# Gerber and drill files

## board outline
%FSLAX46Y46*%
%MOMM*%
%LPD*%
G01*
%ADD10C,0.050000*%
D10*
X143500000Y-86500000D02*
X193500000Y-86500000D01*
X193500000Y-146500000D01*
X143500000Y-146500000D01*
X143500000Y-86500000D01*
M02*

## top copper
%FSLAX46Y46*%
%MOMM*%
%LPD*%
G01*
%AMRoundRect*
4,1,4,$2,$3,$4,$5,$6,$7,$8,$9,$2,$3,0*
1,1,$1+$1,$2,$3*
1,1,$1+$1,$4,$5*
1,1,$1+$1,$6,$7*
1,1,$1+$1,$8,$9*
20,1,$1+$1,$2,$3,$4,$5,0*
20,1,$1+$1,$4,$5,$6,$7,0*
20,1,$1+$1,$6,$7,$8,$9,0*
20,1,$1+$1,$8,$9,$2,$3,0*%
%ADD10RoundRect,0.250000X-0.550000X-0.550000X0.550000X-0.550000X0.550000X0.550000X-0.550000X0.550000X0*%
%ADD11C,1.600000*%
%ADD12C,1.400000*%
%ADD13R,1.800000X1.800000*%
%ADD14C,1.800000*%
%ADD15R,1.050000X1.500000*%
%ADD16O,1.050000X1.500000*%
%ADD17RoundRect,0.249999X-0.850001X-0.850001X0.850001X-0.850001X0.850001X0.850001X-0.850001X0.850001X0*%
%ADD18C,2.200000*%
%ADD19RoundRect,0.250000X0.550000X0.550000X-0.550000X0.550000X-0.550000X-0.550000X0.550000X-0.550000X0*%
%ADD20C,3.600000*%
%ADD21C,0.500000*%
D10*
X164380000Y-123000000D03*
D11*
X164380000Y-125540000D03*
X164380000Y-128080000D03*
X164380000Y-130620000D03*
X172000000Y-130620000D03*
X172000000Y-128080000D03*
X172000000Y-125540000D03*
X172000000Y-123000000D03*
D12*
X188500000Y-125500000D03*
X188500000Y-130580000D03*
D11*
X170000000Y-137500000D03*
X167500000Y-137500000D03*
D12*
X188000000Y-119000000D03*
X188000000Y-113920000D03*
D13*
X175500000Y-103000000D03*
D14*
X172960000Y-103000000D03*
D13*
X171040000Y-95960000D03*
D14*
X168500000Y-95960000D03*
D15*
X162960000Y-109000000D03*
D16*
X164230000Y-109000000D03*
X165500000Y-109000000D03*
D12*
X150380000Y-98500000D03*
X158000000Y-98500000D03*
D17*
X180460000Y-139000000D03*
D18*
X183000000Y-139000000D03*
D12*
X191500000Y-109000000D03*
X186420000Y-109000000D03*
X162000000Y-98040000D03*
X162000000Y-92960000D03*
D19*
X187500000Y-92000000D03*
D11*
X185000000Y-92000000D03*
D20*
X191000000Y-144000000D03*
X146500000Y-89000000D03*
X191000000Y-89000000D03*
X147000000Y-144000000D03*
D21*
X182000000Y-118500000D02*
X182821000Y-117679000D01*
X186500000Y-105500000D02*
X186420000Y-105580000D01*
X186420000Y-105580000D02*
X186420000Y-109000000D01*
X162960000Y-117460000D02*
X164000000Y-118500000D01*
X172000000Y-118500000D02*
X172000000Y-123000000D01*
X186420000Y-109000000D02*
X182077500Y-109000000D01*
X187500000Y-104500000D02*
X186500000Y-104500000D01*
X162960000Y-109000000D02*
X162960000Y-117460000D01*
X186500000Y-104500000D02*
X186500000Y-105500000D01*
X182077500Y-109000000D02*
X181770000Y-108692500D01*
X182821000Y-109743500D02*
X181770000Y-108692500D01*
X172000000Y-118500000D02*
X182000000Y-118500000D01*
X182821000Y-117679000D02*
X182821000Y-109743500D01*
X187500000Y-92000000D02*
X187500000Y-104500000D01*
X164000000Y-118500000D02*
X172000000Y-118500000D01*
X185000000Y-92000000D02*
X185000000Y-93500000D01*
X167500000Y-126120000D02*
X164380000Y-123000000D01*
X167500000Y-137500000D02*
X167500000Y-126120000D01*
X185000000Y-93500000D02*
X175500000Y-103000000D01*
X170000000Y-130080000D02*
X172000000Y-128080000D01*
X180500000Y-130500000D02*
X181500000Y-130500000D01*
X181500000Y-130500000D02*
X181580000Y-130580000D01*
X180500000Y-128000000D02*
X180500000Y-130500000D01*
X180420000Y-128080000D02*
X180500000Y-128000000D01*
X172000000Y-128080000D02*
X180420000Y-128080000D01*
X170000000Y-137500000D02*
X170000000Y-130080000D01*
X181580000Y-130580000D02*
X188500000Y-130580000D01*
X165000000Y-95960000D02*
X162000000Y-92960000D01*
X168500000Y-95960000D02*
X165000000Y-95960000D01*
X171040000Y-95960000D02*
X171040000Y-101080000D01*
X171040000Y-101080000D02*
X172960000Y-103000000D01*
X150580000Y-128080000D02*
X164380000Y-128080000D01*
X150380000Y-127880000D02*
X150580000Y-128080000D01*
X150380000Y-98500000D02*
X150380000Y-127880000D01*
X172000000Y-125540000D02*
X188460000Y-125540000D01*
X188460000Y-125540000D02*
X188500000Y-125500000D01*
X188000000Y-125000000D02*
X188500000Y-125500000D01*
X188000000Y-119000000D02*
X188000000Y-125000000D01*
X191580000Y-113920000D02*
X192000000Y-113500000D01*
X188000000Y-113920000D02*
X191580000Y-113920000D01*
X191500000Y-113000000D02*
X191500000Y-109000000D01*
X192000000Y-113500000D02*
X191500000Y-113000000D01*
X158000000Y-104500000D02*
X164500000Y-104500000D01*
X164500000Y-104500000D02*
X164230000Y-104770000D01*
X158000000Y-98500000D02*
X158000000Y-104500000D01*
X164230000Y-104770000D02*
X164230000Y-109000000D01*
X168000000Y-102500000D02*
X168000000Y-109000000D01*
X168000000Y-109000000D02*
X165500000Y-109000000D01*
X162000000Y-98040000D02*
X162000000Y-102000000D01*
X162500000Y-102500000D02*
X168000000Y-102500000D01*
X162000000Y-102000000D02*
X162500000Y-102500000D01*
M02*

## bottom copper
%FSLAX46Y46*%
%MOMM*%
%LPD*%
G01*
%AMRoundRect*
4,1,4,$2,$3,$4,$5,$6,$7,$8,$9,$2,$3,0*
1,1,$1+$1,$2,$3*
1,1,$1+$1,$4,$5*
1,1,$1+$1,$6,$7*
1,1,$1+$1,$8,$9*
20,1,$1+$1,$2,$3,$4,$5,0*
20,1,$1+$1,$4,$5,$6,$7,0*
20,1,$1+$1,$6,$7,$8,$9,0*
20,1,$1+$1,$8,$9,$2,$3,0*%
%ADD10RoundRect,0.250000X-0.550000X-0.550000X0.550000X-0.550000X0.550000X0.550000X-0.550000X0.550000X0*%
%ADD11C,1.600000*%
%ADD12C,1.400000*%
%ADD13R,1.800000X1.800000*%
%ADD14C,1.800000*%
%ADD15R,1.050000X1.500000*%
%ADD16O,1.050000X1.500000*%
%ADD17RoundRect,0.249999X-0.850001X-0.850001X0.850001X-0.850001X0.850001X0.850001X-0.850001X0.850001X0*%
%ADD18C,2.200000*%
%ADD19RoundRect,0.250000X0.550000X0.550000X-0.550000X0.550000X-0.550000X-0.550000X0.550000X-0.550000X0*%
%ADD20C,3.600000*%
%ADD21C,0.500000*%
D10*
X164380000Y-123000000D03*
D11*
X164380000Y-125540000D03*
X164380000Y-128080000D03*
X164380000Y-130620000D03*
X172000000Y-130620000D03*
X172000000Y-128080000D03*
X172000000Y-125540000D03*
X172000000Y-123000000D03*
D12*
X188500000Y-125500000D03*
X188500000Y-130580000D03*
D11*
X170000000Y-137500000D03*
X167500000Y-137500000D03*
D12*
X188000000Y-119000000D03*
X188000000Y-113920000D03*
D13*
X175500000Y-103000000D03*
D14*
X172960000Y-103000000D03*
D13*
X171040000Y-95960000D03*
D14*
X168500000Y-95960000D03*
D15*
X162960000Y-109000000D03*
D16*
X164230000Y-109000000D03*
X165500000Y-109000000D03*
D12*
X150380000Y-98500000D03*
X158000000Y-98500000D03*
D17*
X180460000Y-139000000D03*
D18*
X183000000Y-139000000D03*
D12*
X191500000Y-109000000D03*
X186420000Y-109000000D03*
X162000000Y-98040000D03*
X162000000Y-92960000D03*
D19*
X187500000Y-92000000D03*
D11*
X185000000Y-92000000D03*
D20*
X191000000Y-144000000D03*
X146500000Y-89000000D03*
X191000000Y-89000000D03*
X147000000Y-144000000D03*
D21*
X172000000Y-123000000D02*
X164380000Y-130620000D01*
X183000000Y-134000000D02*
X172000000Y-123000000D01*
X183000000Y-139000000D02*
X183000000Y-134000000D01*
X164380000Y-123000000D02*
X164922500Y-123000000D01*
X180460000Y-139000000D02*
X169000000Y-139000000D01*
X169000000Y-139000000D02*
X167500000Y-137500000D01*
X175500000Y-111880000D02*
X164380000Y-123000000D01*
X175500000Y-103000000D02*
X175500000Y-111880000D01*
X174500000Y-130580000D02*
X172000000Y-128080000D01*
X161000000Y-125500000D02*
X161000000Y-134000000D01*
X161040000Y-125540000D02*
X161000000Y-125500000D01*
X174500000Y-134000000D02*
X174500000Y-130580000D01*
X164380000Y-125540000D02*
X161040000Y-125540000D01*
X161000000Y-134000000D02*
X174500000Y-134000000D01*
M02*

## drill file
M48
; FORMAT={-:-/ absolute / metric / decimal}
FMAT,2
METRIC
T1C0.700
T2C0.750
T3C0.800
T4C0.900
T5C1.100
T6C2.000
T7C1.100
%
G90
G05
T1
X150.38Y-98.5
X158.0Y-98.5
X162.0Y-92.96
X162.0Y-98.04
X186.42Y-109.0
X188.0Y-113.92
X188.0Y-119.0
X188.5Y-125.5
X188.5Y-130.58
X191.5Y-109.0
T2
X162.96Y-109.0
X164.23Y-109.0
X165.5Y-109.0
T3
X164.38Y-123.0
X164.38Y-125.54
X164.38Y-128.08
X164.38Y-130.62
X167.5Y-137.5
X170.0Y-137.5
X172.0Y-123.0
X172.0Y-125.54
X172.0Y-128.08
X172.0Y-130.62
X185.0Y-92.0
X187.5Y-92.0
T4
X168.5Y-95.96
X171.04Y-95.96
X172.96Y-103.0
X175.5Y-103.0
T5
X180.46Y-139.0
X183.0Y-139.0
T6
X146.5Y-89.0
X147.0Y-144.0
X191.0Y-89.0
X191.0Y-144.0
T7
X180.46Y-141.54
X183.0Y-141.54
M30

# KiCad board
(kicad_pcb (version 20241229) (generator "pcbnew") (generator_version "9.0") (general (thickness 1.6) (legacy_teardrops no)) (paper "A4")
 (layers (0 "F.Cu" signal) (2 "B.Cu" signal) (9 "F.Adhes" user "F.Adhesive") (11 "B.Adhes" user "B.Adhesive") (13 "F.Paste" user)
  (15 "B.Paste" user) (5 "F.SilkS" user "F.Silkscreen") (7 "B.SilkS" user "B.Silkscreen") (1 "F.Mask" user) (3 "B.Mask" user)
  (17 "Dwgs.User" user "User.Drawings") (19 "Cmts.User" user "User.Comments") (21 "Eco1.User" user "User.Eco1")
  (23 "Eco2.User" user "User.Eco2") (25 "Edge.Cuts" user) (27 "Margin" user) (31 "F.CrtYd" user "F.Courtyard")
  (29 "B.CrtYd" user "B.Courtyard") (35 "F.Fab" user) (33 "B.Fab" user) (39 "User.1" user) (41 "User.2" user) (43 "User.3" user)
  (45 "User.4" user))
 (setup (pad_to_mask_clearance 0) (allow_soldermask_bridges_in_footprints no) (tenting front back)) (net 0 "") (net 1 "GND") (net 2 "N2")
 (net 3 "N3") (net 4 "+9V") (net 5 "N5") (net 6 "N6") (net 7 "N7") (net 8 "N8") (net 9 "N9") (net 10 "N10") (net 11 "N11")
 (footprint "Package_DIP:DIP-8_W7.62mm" (layer "F.Cu") (at 164.38 123)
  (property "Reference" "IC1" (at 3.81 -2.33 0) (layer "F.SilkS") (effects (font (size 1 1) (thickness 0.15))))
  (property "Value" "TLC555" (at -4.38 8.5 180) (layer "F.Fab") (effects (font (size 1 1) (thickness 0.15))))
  (pad "1" thru_hole roundrect (at 0 0) (size 1.6 1.6) (drill 0.8) (layers "*.Cu" "*.Mask") (remove_unused_layers no)
   (roundrect_rratio 0.15625) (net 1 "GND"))
  (pad "2" thru_hole circle (at 0 2.54) (size 1.6 1.6) (drill 0.8) (layers "*.Cu" "*.Mask") (remove_unused_layers no) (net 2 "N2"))
  (pad "3" thru_hole circle (at 0 5.08) (size 1.6 1.6) (drill 0.8) (layers "*.Cu" "*.Mask") (remove_unused_layers no) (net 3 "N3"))
  (pad "4" thru_hole circle (at 0 7.62) (size 1.6 1.6) (drill 0.8) (layers "*.Cu" "*.Mask") (remove_unused_layers no) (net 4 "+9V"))
  (pad "5" thru_hole circle (at 7.62 7.62) (size 1.6 1.6) (drill 0.8) (layers "*.Cu" "*.Mask") (remove_unused_layers no) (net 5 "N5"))
  (pad "6" thru_hole circle (at 7.62 5.08) (size 1.6 1.6) (drill 0.8) (layers "*.Cu" "*.Mask") (remove_unused_layers no) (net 2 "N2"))
  (pad "7" thru_hole circle (at 7.62 2.54) (size 1.6 1.6) (drill 0.8) (layers "*.Cu" "*.Mask") (remove_unused_layers no) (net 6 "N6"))
  (pad "8" thru_hole circle (at 7.62 0) (size 1.6 1.6) (drill 0.8) (layers "*.Cu" "*.Mask") (remove_unused_layers no) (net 4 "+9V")))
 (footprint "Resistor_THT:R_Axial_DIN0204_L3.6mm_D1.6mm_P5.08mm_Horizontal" (layer "F.Cu") (at 188.5 125.5 -90)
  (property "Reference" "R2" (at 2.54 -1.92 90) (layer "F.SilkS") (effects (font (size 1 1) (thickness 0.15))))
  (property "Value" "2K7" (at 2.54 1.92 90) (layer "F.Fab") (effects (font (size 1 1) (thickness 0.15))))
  (pad "1" thru_hole circle (at 0 0 270) (size 1.4 1.4) (drill 0.7) (layers "*.Cu" "*.Mask") (remove_unused_layers no) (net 6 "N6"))
  (pad "2" thru_hole circle (at 5.08 0 270) (size 1.4 1.4) (drill 0.7) (layers "*.Cu" "*.Mask") (remove_unused_layers no) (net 2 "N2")))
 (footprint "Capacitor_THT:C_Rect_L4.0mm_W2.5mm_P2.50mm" (layer "F.Cu") (at 170 137.5 180)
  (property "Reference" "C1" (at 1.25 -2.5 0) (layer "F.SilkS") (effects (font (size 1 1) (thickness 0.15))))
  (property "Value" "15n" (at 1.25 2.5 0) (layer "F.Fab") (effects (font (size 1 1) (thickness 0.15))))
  (pad "1" thru_hole circle (at 0 0 180) (size 1.6 1.6) (drill 0.8) (layers "*.Cu" "*.Mask") (remove_unused_layers no) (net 2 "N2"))
  (pad "2" thru_hole circle (at 2.5 0 180) (size 1.6 1.6) (drill 0.8) (layers "*.Cu" "*.Mask") (remove_unused_layers no) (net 1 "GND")))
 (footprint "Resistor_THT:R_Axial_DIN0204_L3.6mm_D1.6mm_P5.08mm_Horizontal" (layer "F.Cu") (at 188 119 90)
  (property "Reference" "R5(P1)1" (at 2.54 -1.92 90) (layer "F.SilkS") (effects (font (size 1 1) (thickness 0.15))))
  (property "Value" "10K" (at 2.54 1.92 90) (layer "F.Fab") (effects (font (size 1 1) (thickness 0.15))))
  (pad "1" thru_hole circle (at 0 0 90) (size 1.4 1.4) (drill 0.7) (layers "*.Cu" "*.Mask") (remove_unused_layers no) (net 6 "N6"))
  (pad "2" thru_hole circle (at 5.08 0 90) (size 1.4 1.4) (drill 0.7) (layers "*.Cu" "*.Mask") (remove_unused_layers no) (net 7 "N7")))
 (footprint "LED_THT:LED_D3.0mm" (layer "F.Cu") (at 175.5 103 180)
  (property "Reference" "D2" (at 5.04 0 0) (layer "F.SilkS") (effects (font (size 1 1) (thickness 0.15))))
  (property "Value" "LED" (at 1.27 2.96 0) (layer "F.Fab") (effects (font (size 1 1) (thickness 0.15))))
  (pad "1" thru_hole rect (at 0 0 180) (size 1.8 1.8) (drill 0.9) (layers "*.Cu" "*.Mask") (remove_unused_layers no) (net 1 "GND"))
  (pad "2" thru_hole circle (at 2.54 0 180) (size 1.8 1.8) (drill 0.9) (layers "*.Cu" "*.Mask") (remove_unused_layers no) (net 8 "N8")))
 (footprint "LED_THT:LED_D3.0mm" (layer "F.Cu") (at 171.04 95.96 180)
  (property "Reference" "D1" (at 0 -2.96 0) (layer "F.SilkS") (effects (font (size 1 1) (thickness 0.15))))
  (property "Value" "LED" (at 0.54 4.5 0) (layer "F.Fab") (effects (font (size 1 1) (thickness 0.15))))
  (pad "1" thru_hole rect (at 0 0 180) (size 1.8 1.8) (drill 0.9) (layers "*.Cu" "*.Mask") (remove_unused_layers no) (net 8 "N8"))
  (pad "2" thru_hole circle (at 2.54 0 180) (size 1.8 1.8) (drill 0.9) (layers "*.Cu" "*.Mask") (remove_unused_layers no) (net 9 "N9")))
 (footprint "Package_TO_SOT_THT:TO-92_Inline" (layer "F.Cu") (at 162.96 109)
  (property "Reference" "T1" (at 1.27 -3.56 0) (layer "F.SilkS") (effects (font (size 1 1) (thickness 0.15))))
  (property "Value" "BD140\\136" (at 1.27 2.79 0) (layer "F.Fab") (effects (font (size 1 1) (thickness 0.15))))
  (pad "1" thru_hole rect (at 0 0) (size 1.05 1.5) (drill 0.75) (layers "*.Cu" "*.Mask") (remove_unused_layers no) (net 4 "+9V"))
  (pad "2" thru_hole oval (at 1.27 0) (size 1.05 1.5) (drill 0.75) (layers "*.Cu" "*.Mask") (remove_unused_layers no) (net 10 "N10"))
  (pad "3" thru_hole oval (at 2.54 0) (size 1.05 1.5) (drill 0.75) (layers "*.Cu" "*.Mask") (remove_unused_layers no) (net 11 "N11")))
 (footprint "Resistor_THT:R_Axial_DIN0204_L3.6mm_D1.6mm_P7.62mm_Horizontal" (layer "F.Cu") (at 150.38 98.5)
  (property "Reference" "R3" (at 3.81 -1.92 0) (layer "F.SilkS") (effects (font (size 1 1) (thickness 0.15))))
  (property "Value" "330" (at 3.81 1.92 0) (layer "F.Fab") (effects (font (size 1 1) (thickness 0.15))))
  (pad "1" thru_hole circle (at 0 0) (size 1.4 1.4) (drill 0.7) (layers "*.Cu" "*.Mask") (remove_unused_layers no) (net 3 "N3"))
  (pad "2" thru_hole circle (at 7.62 0) (size 1.4 1.4) (drill 0.7) (layers "*.Cu" "*.Mask") (remove_unused_layers no) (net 10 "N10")))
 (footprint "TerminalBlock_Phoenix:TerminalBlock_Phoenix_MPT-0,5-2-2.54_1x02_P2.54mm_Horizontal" (layer "F.Cu") (at 180.46 139)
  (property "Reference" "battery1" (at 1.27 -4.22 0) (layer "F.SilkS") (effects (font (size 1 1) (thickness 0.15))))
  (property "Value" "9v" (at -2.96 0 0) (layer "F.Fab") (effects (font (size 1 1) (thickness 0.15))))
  (pad "" np_thru_hole circle (at 0 2.54) (size 1.1 1.1) (drill 1.1) (layers "*.Cu" "*.Mask"))
  (pad "" np_thru_hole circle (at 2.54 2.54) (size 1.1 1.1) (drill 1.1) (layers "*.Cu" "*.Mask"))
  (pad "1" thru_hole roundrect (at 0 0) (size 2.2 2.2) (drill 1.1) (layers "*.Cu" "*.Mask") (remove_unused_layers no)
   (roundrect_rratio 0.113636) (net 1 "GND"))
  (pad "2" thru_hole circle (at 2.54 0) (size 2.2 2.2) (drill 1.1) (layers "*.Cu" "*.Mask") (remove_unused_layers no) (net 4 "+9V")))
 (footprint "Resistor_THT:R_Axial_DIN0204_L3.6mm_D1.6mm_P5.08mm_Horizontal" (layer "F.Cu") (at 191.5 109 180)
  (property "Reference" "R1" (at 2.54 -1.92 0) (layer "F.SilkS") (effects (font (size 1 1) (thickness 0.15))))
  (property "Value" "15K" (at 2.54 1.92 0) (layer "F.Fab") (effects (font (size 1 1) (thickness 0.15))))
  (pad "1" thru_hole circle (at 0 0 180) (size 1.4 1.4) (drill 0.7) (layers "*.Cu" "*.Mask") (remove_unused_layers no) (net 7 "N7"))
  (pad "2" thru_hole circle (at 5.08 0 180) (size 1.4 1.4) (drill 0.7) (layers "*.Cu" "*.Mask") (remove_unused_layers no) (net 4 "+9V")))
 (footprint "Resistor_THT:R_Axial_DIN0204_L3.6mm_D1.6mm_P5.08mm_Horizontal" (layer "F.Cu") (at 162 98.04 90)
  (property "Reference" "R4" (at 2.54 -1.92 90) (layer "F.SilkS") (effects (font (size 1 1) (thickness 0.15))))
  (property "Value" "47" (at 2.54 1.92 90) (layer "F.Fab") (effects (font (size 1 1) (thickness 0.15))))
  (pad "1" thru_hole circle (at 0 0 90) (size 1.4 1.4) (drill 0.7) (layers "*.Cu" "*.Mask") (remove_unused_layers no) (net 11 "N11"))
  (pad "2" thru_hole circle (at 5.08 0 90) (size 1.4 1.4) (drill 0.7) (layers "*.Cu" "*.Mask") (remove_unused_layers no) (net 9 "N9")))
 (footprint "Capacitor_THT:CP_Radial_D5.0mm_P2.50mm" (layer "F.Cu") (at 187.5 92 180)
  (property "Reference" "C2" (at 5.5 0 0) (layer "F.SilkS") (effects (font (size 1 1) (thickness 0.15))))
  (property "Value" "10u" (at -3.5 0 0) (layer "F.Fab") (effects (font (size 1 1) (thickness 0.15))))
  (pad "1" thru_hole roundrect (at 0 0 180) (size 1.6 1.6) (drill 0.8) (layers "*.Cu" "*.Mask") (remove_unused_layers no)
   (roundrect_rratio 0.15625) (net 4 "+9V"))
  (pad "2" thru_hole circle (at 2.5 0 180) (size 1.6 1.6) (drill 0.8) (layers "*.Cu" "*.Mask") (remove_unused_layers no) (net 1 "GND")))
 (gr_rect (start 143.5 86.5) (end 193.5 146.5) (stroke (width 0.05) (type default)) (fill no) (layer "Edge.Cuts"))
 (via (at 191 144) (size 3.6) (drill 2) (layers "F.Cu" "B.Cu") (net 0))
 (via (at 146.5 89) (size 3.6) (drill 2) (layers "F.Cu" "B.Cu") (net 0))
 (via (at 191 89) (size 3.6) (drill 2) (layers "F.Cu" "B.Cu") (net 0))
 (via (at 147 144) (size 3.6) (drill 2) (layers "F.Cu" "B.Cu") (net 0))
 (segment (start 182 118.5) (end 182.821 117.679) (width 0.5) (layer "F.Cu") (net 4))
 (segment (start 186.5 105.5) (end 186.42 105.58) (width 0.5) (layer "F.Cu") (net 4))
 (segment (start 186.42 105.58) (end 186.42 109) (width 0.5) (layer "F.Cu") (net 4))
 (segment (start 162.96 117.46) (end 164 118.5) (width 0.5) (layer "F.Cu") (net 4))
 (segment (start 172 118.5) (end 172 123) (width 0.5) (layer "F.Cu") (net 4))
 (segment (start 186.42 109) (end 182.0775 109) (width 0.5) (layer "F.Cu") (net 4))
 (segment (start 187.5 104.5) (end 186.5 104.5) (width 0.5) (layer "F.Cu") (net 4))
 (segment (start 162.96 109) (end 162.96 117.46) (width 0.5) (layer "F.Cu") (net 4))
 (segment (start 186.5 104.5) (end 186.5 105.5) (width 0.5) (layer "F.Cu") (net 4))
 (segment (start 182.0775 109) (end 181.77 108.6925) (width 0.5) (layer "F.Cu") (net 4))
 (segment (start 182.821 109.7435) (end 181.77 108.6925) (width 0.5) (layer "F.Cu") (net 4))
 (segment (start 172 118.5) (end 182 118.5) (width 0.5) (layer "F.Cu") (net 4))
 (segment (start 182.821 117.679) (end 182.821 109.7435) (width 0.5) (layer "F.Cu") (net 4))
 (segment (start 187.5 92) (end 187.5 104.5) (width 0.5) (layer "F.Cu") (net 4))
 (segment (start 164 118.5) (end 172 118.5) (width 0.5) (layer "F.Cu") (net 4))
 (segment (start 172 123) (end 164.38 130.62) (width 0.5) (layer "B.Cu") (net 4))
 (segment (start 183 134) (end 172 123) (width 0.5) (layer "B.Cu") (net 4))
 (segment (start 183 139) (end 183 134) (width 0.5) (layer "B.Cu") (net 4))
 (segment (start 185 92) (end 185 93.5) (width 0.5) (layer "F.Cu") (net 1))
 (segment (start 167.5 126.12) (end 164.38 123) (width 0.5) (layer "F.Cu") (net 1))
 (segment (start 167.5 137.5) (end 167.5 126.12) (width 0.5) (layer "F.Cu") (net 1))
 (segment (start 185 93.5) (end 175.5 103) (width 0.5) (layer "F.Cu") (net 1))
 (segment (start 164.38 123) (end 164.9225 123) (width 0.5) (layer "B.Cu") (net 1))
 (segment (start 180.46 139) (end 169 139) (width 0.5) (layer "B.Cu") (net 1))
 (segment (start 169 139) (end 167.5 137.5) (width 0.5) (layer "B.Cu") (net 1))
 (segment (start 175.5 111.88) (end 164.38 123) (width 0.5) (layer "B.Cu") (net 1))
 (segment (start 175.5 103) (end 175.5 111.88) (width 0.5) (layer "B.Cu") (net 1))
 (segment (start 170 130.08) (end 172 128.08) (width 0.5) (layer "F.Cu") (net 2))
 (segment (start 180.5 130.5) (end 181.5 130.5) (width 0.5) (layer "F.Cu") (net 2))
 (segment (start 181.5 130.5) (end 181.58 130.58) (width 0.5) (layer "F.Cu") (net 2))
 (segment (start 180.5 128) (end 180.5 130.5) (width 0.5) (layer "F.Cu") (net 2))
 (segment (start 180.42 128.08) (end 180.5 128) (width 0.5) (layer "F.Cu") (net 2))
 (segment (start 172 128.08) (end 180.42 128.08) (width 0.5) (layer "F.Cu") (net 2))
 (segment (start 170 137.5) (end 170 130.08) (width 0.5) (layer "F.Cu") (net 2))
 (segment (start 181.58 130.58) (end 188.5 130.58) (width 0.5) (layer "F.Cu") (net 2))
 (segment (start 174.5 130.58) (end 172 128.08) (width 0.5) (layer "B.Cu") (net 2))
 (segment (start 161 125.5) (end 161 134) (width 0.5) (layer "B.Cu") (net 2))
 (segment (start 161.04 125.54) (end 161 125.5) (width 0.5) (layer "B.Cu") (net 2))
 (segment (start 174.5 134) (end 174.5 130.58) (width 0.5) (layer "B.Cu") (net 2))
 (segment (start 164.38 125.54) (end 161.04 125.54) (width 0.5) (layer "B.Cu") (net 2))
 (segment (start 161 134) (end 174.5 134) (width 0.5) (layer "B.Cu") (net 2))
 (segment (start 165 95.96) (end 162 92.96) (width 0.5) (layer "F.Cu") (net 9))
 (segment (start 168.5 95.96) (end 165 95.96) (width 0.5) (layer "F.Cu") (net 9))
 (segment (start 171.04 95.96) (end 171.04 101.08) (width 0.5) (layer "F.Cu") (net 8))
 (segment (start 171.04 101.08) (end 172.96 103) (width 0.5) (layer "F.Cu") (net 8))
 (segment (start 150.58 128.08) (end 164.38 128.08) (width 0.5) (layer "F.Cu") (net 3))
 (segment (start 150.38 127.88) (end 150.58 128.08) (width 0.5) (layer "F.Cu") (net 3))
 (segment (start 150.38 98.5) (end 150.38 127.88) (width 0.5) (layer "F.Cu") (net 3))
 (segment (start 172 125.54) (end 188.46 125.54) (width 0.5) (layer "F.Cu") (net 6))
 (segment (start 188.46 125.54) (end 188.5 125.5) (width 0.5) (layer "F.Cu") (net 6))
 (segment (start 188 125) (end 188.5 125.5) (width 0.5) (layer "F.Cu") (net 6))
 (segment (start 188 119) (end 188 125) (width 0.5) (layer "F.Cu") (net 6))
 (segment (start 191.58 113.92) (end 192 113.5) (width 0.5) (layer "F.Cu") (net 7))
 (segment (start 188 113.92) (end 191.58 113.92) (width 0.5) (layer "F.Cu") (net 7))
 (segment (start 191.5 113) (end 191.5 109) (width 0.5) (layer "F.Cu") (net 7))
 (segment (start 192 113.5) (end 191.5 113) (width 0.5) (layer "F.Cu") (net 7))
 (segment (start 158 104.5) (end 164.5 104.5) (width 0.5) (layer "F.Cu") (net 10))
 (segment (start 164.5 104.5) (end 164.23 104.77) (width 0.5) (layer "F.Cu") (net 10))
 (segment (start 158 98.5) (end 158 104.5) (width 0.5) (layer "F.Cu") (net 10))
 (segment (start 164.23 104.77) (end 164.23 109) (width 0.5) (layer "F.Cu") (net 10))
 (segment (start 168 102.5) (end 168 109) (width 0.5) (layer "F.Cu") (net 11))
 (segment (start 168 109) (end 165.5 109) (width 0.5) (layer "F.Cu") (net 11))
 (segment (start 162 98.04) (end 162 102) (width 0.5) (layer "F.Cu") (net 11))
 (segment (start 162.5 102.5) (end 168 102.5) (width 0.5) (layer "F.Cu") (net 11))
 (segment (start 162 102) (end 162.5 102.5) (width 0.5) (layer "F.Cu") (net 11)))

